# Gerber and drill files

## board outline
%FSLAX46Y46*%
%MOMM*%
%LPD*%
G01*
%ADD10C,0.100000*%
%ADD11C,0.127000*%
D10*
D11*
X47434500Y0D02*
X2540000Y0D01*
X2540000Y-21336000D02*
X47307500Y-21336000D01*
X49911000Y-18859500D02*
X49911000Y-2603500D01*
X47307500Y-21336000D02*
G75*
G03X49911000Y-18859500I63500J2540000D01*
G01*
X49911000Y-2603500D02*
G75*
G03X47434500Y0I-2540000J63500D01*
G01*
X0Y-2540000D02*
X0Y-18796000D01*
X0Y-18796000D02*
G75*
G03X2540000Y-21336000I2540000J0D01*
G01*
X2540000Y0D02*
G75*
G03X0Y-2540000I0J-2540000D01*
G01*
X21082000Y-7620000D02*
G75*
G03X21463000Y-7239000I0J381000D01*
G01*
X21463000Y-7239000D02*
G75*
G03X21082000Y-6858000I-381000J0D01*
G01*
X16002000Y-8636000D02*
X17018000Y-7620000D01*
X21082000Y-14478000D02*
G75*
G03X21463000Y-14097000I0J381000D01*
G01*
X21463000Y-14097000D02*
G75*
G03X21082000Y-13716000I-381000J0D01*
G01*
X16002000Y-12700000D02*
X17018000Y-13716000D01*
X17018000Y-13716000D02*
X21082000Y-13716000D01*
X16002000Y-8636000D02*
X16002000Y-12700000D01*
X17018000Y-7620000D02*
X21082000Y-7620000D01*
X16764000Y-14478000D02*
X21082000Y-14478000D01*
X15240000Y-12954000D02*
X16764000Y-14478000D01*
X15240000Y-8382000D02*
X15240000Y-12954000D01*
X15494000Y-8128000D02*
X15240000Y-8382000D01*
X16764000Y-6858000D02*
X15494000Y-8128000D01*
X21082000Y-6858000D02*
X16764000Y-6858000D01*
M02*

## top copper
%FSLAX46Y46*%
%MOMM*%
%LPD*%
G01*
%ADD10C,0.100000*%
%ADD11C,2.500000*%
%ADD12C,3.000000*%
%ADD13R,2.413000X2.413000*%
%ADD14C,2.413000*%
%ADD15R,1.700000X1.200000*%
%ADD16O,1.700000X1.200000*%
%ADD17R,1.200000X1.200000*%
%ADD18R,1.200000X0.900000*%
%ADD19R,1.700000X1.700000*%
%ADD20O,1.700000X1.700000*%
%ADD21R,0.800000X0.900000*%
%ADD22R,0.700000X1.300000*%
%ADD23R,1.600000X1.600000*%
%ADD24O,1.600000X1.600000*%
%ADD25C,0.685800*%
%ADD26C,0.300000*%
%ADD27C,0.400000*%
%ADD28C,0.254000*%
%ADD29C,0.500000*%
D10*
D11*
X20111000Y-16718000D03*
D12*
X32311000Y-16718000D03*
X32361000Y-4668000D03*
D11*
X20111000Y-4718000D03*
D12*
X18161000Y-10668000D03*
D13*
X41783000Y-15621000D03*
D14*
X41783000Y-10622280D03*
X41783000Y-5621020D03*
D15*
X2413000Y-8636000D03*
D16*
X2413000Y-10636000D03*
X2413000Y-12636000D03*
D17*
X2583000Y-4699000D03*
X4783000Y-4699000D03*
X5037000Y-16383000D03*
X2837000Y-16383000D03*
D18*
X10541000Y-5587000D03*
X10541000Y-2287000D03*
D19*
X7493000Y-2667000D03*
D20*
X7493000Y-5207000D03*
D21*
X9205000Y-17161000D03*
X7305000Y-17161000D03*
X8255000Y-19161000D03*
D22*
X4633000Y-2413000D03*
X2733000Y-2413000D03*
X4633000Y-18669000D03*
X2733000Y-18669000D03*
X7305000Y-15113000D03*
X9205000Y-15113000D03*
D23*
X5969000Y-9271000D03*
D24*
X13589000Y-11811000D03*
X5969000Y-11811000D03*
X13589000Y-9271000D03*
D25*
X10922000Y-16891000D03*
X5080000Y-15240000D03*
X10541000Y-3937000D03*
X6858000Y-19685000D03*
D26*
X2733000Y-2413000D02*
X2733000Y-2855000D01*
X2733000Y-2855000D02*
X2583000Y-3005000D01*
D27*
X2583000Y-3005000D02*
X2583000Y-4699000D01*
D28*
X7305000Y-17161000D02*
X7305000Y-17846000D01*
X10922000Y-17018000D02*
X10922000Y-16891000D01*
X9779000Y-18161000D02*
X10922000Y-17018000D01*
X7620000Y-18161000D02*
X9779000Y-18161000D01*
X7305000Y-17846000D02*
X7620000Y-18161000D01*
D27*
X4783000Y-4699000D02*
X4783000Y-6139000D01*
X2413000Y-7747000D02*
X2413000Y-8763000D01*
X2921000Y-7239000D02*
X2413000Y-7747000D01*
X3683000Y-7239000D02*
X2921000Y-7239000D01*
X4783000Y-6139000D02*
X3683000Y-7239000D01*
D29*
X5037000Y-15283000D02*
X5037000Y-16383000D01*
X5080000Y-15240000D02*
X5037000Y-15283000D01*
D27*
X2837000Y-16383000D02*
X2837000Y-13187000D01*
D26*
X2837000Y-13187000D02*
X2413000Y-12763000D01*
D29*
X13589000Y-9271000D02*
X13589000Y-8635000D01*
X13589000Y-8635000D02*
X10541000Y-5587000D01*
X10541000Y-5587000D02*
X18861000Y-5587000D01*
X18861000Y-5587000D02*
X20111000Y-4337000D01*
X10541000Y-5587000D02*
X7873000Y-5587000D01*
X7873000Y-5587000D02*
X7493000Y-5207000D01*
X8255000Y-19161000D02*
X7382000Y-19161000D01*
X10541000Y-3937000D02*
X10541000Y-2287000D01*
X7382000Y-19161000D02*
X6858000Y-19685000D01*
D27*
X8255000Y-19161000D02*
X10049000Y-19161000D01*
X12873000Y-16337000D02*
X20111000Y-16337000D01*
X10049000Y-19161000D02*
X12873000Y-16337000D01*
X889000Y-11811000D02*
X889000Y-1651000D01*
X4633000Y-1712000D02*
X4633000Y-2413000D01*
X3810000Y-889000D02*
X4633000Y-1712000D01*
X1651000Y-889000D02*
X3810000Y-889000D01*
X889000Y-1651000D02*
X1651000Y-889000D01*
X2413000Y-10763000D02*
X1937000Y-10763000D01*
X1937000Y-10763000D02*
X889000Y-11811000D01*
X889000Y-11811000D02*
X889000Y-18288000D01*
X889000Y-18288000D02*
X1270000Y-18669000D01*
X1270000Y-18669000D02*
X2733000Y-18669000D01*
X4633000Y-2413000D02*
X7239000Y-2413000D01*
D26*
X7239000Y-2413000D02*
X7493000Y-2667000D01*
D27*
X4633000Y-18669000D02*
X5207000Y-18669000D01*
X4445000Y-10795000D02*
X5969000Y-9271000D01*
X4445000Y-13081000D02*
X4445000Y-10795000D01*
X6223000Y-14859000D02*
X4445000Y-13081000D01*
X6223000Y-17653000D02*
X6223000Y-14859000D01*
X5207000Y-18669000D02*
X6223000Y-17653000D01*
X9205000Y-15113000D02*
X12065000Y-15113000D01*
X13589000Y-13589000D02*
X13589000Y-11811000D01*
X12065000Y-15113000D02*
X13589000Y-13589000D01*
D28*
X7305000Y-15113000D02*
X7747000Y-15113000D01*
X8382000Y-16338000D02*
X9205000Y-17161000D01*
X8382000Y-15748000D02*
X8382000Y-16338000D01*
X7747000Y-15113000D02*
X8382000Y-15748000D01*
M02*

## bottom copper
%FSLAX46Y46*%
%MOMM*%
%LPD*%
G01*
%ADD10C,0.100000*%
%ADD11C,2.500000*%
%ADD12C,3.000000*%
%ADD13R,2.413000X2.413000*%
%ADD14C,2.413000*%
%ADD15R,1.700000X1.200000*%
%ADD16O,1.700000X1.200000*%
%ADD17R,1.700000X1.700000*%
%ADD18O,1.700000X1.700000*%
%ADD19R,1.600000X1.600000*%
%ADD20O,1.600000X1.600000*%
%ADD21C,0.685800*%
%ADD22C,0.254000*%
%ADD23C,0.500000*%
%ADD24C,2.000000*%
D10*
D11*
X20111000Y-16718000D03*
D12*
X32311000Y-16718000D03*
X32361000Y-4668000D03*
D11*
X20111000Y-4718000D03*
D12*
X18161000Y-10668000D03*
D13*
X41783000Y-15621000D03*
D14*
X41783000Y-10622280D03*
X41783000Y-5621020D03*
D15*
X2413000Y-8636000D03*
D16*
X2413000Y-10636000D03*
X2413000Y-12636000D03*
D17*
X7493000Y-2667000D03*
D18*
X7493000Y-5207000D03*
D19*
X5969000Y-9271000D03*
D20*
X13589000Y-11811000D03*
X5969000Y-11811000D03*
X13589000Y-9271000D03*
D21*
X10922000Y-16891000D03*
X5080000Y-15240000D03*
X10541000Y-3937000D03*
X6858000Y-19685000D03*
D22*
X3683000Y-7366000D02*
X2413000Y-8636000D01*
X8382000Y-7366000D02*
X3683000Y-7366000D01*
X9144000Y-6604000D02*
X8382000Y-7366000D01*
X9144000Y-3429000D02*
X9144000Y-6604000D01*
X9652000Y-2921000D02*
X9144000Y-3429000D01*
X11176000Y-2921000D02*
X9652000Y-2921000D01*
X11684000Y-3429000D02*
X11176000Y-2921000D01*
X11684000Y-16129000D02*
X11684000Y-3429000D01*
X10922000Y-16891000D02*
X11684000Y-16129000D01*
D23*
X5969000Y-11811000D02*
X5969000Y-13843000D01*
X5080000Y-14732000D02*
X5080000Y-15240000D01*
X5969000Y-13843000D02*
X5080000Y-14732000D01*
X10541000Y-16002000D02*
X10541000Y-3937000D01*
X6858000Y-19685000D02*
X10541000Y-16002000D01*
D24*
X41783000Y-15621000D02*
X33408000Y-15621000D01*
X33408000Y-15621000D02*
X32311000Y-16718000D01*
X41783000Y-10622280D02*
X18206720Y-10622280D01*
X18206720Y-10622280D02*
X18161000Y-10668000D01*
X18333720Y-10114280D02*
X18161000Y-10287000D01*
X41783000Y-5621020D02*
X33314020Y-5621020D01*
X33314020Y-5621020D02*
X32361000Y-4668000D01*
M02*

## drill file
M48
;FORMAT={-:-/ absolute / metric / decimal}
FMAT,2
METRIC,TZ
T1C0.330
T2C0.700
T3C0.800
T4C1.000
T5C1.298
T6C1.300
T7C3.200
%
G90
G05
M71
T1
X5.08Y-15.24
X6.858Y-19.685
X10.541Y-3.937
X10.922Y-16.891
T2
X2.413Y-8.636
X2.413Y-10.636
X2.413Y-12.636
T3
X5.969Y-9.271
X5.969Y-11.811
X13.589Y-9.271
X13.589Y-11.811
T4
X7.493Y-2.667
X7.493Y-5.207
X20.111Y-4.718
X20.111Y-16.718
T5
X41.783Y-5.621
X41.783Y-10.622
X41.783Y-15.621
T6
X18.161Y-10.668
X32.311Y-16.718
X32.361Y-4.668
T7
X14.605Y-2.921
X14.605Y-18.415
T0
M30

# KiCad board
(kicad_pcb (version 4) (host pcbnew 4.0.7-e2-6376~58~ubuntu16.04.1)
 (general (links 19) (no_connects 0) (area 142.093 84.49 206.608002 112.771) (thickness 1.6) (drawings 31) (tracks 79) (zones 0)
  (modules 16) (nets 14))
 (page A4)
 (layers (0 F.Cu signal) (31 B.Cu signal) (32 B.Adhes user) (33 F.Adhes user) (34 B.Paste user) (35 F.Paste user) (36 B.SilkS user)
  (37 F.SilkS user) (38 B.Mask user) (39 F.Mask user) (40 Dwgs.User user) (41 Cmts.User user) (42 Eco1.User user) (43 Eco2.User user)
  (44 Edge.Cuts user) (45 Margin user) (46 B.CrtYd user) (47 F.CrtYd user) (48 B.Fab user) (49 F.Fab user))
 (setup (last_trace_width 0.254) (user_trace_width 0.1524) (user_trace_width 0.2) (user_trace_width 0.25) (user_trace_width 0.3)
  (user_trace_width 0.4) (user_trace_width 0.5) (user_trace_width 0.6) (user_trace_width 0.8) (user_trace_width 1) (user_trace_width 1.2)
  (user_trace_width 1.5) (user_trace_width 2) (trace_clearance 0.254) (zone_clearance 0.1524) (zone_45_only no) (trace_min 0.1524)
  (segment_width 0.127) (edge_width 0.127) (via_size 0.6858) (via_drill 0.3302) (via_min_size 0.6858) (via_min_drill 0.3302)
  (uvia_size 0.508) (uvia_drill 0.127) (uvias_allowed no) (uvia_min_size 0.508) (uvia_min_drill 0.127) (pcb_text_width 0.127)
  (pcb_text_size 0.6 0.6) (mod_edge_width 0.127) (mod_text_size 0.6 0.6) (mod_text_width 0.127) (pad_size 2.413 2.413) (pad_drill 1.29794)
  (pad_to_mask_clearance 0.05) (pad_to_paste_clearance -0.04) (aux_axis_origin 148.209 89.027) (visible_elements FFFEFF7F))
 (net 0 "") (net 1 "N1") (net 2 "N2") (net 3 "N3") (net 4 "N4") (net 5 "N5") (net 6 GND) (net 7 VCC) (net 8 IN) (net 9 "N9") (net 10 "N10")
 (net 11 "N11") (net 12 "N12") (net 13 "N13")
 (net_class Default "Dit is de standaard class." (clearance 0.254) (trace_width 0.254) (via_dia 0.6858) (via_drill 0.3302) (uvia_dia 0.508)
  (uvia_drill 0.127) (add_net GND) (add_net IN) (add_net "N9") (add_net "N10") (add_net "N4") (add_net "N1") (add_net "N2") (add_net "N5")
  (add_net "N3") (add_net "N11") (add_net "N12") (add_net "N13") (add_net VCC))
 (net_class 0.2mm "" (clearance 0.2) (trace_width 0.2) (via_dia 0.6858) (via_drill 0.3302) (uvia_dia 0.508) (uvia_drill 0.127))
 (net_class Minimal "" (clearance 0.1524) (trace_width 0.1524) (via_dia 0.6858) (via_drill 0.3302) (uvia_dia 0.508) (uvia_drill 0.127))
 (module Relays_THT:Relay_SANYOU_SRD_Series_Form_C (layer F.Cu) (at 166.37 99.695)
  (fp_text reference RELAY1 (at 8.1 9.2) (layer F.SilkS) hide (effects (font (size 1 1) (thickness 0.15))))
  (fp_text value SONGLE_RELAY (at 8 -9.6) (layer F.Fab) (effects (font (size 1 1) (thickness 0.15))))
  (pad 4 thru_hole circle (at 1.95 6.05 90) (size 2.5 2.5) (drill 1) (layers *.Cu *.Mask) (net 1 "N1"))
  (pad 1 thru_hole circle (at 14.15 6.05 90) (size 3 3) (drill 1.3) (layers *.Cu *.Mask) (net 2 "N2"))
  (pad 2 thru_hole circle (at 14.2 -6 90) (size 3 3) (drill 1.3) (layers *.Cu *.Mask) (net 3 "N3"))
  (pad 5 thru_hole circle (at 1.95 -5.95 90) (size 2.5 2.5) (drill 1) (layers *.Cu *.Mask) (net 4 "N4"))
  (pad 3 thru_hole circle (at 0 0 90) (size 3 3) (drill 1.3) (layers *.Cu *.Mask) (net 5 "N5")))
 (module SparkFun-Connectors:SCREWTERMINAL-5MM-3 (layer F.Cu) (at 189.992 104.648 90)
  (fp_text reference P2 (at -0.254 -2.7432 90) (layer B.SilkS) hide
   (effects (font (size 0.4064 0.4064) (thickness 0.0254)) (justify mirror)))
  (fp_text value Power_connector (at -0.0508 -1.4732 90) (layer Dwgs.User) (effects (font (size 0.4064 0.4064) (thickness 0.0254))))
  (pad 1 thru_hole rect (at 0 0 90) (size 2.413 2.413) (drill 1.29794) (layers *.Cu *.Mask F.Paste F.SilkS) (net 2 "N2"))
  (pad 2 thru_hole circle (at 4.99872 0 90) (size 2.413 2.413) (drill 1.29794) (layers *.Cu *.Mask F.Paste F.SilkS) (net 5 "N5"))
  (pad 3 thru_hole circle (at 9.99998 0 90) (size 2.413 2.413) (drill 1.29794) (layers *.Cu *.Mask F.Paste F.SilkS) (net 3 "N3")))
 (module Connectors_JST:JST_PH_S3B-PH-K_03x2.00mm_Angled (layer F.Cu) (at 150.622 97.663 270)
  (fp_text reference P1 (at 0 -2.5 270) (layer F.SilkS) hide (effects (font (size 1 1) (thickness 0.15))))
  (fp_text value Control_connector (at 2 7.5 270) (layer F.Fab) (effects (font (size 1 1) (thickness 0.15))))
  (pad 1 thru_hole rect (at 0 0 270) (size 1.2 1.7) (drill 0.7) (layers *.Cu *.Mask) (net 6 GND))
  (pad 2 thru_hole oval (at 2 0 270) (size 1.2 1.7) (drill 0.7) (layers *.Cu *.Mask) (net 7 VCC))
  (pad 3 thru_hole oval (at 4 0 270) (size 1.2 1.7) (drill 0.7) (layers *.Cu *.Mask) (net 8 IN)))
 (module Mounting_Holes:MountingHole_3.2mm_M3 (layer F.Cu) (at 162.814 107.442)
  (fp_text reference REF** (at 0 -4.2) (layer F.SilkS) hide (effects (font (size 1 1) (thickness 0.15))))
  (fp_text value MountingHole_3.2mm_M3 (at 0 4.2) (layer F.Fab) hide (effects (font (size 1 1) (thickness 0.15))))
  (pad 1 np_thru_hole circle (at 0 0) (size 3.2 3.2) (drill 3.2) (layers *.Cu *.Mask)))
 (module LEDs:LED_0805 (layer F.Cu) (at 151.892 93.726 180)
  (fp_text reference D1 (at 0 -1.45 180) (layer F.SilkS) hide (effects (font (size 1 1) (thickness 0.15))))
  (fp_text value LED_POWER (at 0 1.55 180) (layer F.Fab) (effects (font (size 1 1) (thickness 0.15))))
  (pad 2 smd rect (at 1.1 0) (size 1.2 1.2) (layers F.Cu F.Paste F.Mask) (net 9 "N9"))
  (pad 1 smd rect (at -1.1 0) (size 1.2 1.2) (layers F.Cu F.Paste F.Mask) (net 6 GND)))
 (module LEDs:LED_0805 (layer F.Cu) (at 152.146 105.41)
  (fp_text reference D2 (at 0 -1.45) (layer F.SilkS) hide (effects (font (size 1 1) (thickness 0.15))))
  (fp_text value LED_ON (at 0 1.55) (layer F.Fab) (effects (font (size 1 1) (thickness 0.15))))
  (pad 2 smd rect (at 1.1 0 180) (size 1.2 1.2) (layers F.Cu F.Paste F.Mask) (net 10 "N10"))
  (pad 1 smd rect (at -1.1 0 180) (size 1.2 1.2) (layers F.Cu F.Paste F.Mask) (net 8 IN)))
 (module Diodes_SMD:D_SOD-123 (layer F.Cu) (at 158.75 92.964 90)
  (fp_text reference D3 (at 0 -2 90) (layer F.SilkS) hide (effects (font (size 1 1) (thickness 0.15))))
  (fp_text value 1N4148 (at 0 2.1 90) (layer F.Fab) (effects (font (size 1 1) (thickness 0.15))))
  (pad 1 smd rect (at -1.65 0 90) (size 0.9 1.2) (layers F.Cu F.Paste F.Mask) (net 4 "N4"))
  (pad 2 smd rect (at 1.65 0 90) (size 0.9 1.2) (layers F.Cu F.Paste F.Mask) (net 1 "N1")))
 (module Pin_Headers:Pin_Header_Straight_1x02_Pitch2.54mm (layer F.Cu) (at 155.702 91.694)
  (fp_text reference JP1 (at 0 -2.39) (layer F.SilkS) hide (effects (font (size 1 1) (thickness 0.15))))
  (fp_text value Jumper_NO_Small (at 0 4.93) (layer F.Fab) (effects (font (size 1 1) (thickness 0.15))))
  (pad 1 thru_hole rect (at 0 0) (size 1.7 1.7) (drill 1) (layers *.Cu *.Mask) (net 7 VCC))
  (pad 2 thru_hole oval (at 0 2.54) (size 1.7 1.7) (drill 1) (layers *.Cu *.Mask) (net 4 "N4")))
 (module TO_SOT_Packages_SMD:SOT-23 (layer F.Cu) (at 156.464 107.188 270)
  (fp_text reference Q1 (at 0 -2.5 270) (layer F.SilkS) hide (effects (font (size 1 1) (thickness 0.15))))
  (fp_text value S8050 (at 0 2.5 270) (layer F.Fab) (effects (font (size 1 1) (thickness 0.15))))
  (pad 1 smd rect (at -1 -0.95 270) (size 0.9 0.8) (layers F.Cu F.Paste F.Mask) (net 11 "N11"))
  (pad 2 smd rect (at -1 0.95 270) (size 0.9 0.8) (layers F.Cu F.Paste F.Mask) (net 6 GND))
  (pad 3 smd rect (at 1 0 270) (size 0.9 0.8) (layers F.Cu F.Paste F.Mask) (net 1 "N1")))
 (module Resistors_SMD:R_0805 (layer F.Cu) (at 151.892 91.44 180)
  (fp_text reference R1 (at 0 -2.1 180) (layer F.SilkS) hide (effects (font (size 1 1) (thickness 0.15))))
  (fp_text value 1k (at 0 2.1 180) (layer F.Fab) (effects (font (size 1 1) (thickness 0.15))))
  (pad 1 smd rect (at -0.95 0 180) (size 0.7 1.3) (layers F.Cu F.Paste F.Mask) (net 7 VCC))
  (pad 2 smd rect (at 0.95 0 180) (size 0.7 1.3) (layers F.Cu F.Paste F.Mask) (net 9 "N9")))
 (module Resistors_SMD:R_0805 (layer F.Cu) (at 151.892 107.696 180)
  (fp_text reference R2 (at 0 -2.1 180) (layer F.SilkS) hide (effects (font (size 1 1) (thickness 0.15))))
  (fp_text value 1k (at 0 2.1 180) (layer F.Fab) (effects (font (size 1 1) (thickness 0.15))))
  (pad 1 smd rect (at -0.95 0 180) (size 0.7 1.3) (layers F.Cu F.Paste F.Mask) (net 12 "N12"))
  (pad 2 smd rect (at 0.95 0 180) (size 0.7 1.3) (layers F.Cu F.Paste F.Mask) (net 7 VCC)))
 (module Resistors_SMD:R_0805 (layer F.Cu) (at 156.464 104.14)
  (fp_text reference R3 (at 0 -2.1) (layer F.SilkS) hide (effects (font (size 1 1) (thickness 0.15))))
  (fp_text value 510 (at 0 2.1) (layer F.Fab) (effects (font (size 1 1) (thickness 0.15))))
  (pad 1 smd rect (at -0.95 0) (size 0.7 1.3) (layers F.Cu F.Paste F.Mask) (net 11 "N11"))
  (pad 2 smd rect (at 0.95 0) (size 0.7 1.3) (layers F.Cu F.Paste F.Mask) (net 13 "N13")))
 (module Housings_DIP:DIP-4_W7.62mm (layer F.Cu) (at 154.178 98.298)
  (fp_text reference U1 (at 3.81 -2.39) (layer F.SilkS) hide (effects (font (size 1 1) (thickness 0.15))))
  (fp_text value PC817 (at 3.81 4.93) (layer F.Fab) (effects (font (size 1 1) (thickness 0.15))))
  (pad 1 thru_hole rect (at 0 0) (size 1.6 1.6) (drill 0.8) (layers *.Cu *.Mask) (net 12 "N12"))
  (pad 3 thru_hole oval (at 7.62 2.54) (size 1.6 1.6) (drill 0.8) (layers *.Cu *.Mask) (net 13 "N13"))
  (pad 2 thru_hole oval (at 0 2.54) (size 1.6 1.6) (drill 0.8) (layers *.Cu *.Mask) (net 10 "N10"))
  (pad 4 thru_hole oval (at 7.62 0) (size 1.6 1.6) (drill 0.8) (layers *.Cu *.Mask) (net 4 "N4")))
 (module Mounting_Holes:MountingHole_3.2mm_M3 (layer F.Cu) (at 162.814 91.948)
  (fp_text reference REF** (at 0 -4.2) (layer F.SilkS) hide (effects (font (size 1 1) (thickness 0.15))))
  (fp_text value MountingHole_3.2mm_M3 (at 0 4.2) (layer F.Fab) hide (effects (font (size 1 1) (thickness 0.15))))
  (pad 1 np_thru_hole circle (at 0 0) (size 3.2 3.2) (drill 3.2) (layers *.Cu *.Mask)))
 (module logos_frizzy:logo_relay (layer B.Cu) (at 175.26 99.695 90)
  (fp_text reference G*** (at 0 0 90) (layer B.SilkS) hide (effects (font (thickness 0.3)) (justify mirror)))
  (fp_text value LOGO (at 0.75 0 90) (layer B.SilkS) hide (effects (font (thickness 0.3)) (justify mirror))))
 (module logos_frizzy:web (layer F.Cu) (at 174.371 108.712)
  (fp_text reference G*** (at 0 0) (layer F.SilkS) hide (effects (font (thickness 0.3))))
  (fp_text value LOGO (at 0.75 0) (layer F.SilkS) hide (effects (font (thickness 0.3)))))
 (gr_line (start 195.6435 89.027) (end 150.749 89.027) (angle 90) (layer Edge.Cuts) (width 0.127))
 (gr_line (start 150.749 110.363) (end 195.5165 110.363) (angle 90) (layer Edge.Cuts) (width 0.127))
 (gr_line (start 198.12 107.8865) (end 198.12 91.6305) (angle 90) (layer Edge.Cuts) (width 0.127))
 (gr_arc (start 195.58 107.823) (end 198.12 107.8865) (angle 90) (layer Edge.Cuts) (width 0.127))
 (gr_arc (start 195.58 91.567) (end 195.6435 89.027) (angle 90) (layer Edge.Cuts) (width 0.127))
 (gr_line (start 148.209 91.567) (end 148.209 107.823) (angle 90) (layer Edge.Cuts) (width 0.127))
 (gr_arc (start 150.749 107.823) (end 150.749 110.363) (angle 90) (layer Edge.Cuts) (width 0.127))
 (gr_arc (start 150.749 91.567) (end 148.209 91.567) (angle 90) (layer Edge.Cuts) (width 0.127))
 (gr_arc (start 169.291 96.266) (end 169.672 96.266) (angle 90) (layer Edge.Cuts) (width 0.127))
 (gr_arc (start 169.291 96.266) (end 169.291 95.885) (angle 90) (layer Edge.Cuts) (width 0.127))
 (gr_line (start 164.211 97.663) (end 165.227 96.647) (angle 90) (layer Edge.Cuts) (width 0.127))
 (gr_arc (start 169.291 103.124) (end 169.672 103.124) (angle 90) (layer Edge.Cuts) (width 0.127))
 (gr_arc (start 169.291 103.124) (end 169.291 102.743) (angle 90) (layer Edge.Cuts) (width 0.127))
 (gr_line (start 164.211 101.727) (end 165.227 102.743) (angle 90) (layer Edge.Cuts) (width 0.127))
 (gr_line (start 165.227 102.743) (end 169.291 102.743) (angle 90) (layer Edge.Cuts) (width 0.127))
 (gr_line (start 164.211 97.663) (end 164.211 101.727) (angle 90) (layer Edge.Cuts) (width 0.127))
 (gr_line (start 165.227 96.647) (end 169.291 96.647) (angle 90) (layer Edge.Cuts) (width 0.127))
 (gr_line (start 164.973 103.505) (end 169.291 103.505) (angle 90) (layer Edge.Cuts) (width 0.127))
 (gr_line (start 163.449 101.981) (end 164.973 103.505) (angle 90) (layer Edge.Cuts) (width 0.127))
 (gr_line (start 163.449 97.409) (end 163.449 101.981) (angle 90) (layer Edge.Cuts) (width 0.127))
 (gr_line (start 163.703 97.155) (end 163.449 97.409) (angle 90) (layer Edge.Cuts) (width 0.127))
 (gr_line (start 164.973 95.885) (end 163.703 97.155) (angle 90) (layer Edge.Cuts) (width 0.127))
 (gr_line (start 169.291 95.885) (end 164.973 95.885) (angle 90) (layer Edge.Cuts) (width 0.127))
 (segment (start 150.942 91.44) (end 150.942 91.882) (width 0.3) (layer F.Cu) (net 9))
 (segment (start 150.942 91.882) (end 150.792 92.032) (width 0.3) (layer F.Cu) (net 9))
 (segment (start 150.792 92.032) (end 150.792 93.726) (width 0.4) (layer F.Cu) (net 9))
 (segment (start 155.514 106.188) (end 155.514 106.873) (width 0.254) (layer F.Cu) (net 6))
 (segment (start 151.892 96.393) (end 150.622 97.663) (width 0.254) (layer B.Cu) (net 6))
 (segment (start 156.591 96.393) (end 151.892 96.393) (width 0.254) (layer B.Cu) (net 6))
 (segment (start 157.353 95.631) (end 156.591 96.393) (width 0.254) (layer B.Cu) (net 6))
 (segment (start 157.353 92.456) (end 157.353 95.631) (width 0.254) (layer B.Cu) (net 6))
 (segment (start 157.861 91.948) (end 157.353 92.456) (width 0.254) (layer B.Cu) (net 6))
 (segment (start 159.385 91.948) (end 157.861 91.948) (width 0.254) (layer B.Cu) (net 6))
 (segment (start 159.893 92.456) (end 159.385 91.948) (width 0.254) (layer B.Cu) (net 6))
 (segment (start 159.893 105.156) (end 159.893 92.456) (width 0.254) (layer B.Cu) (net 6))
 (segment (start 159.131 105.918) (end 159.893 105.156) (width 0.254) (layer B.Cu) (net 6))
 (via (at 159.131 105.918) (size 0.6858) (drill 0.3302) (layers F.Cu B.Cu) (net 6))
 (segment (start 159.131 106.045) (end 159.131 105.918) (width 0.254) (layer F.Cu) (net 6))
 (segment (start 157.988 107.188) (end 159.131 106.045) (width 0.254) (layer F.Cu) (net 6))
 (segment (start 155.829 107.188) (end 157.988 107.188) (width 0.254) (layer F.Cu) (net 6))
 (segment (start 155.514 106.873) (end 155.829 107.188) (width 0.254) (layer F.Cu) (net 6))
 (segment (start 152.992 93.726) (end 152.992 95.166) (width 0.4) (layer F.Cu) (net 6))
 (segment (start 150.622 96.774) (end 150.622 97.79) (width 0.4) (layer F.Cu) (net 6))
 (segment (start 151.13 96.266) (end 150.622 96.774) (width 0.4) (layer F.Cu) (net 6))
 (segment (start 151.892 96.266) (end 151.13 96.266) (width 0.4) (layer F.Cu) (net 6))
 (segment (start 152.992 95.166) (end 151.892 96.266) (width 0.4) (layer F.Cu) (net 6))
 (segment (start 154.178 100.838) (end 154.178 102.87) (width 0.5) (layer B.Cu) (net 10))
 (segment (start 153.246 104.31) (end 153.246 105.41) (width 0.5) (layer F.Cu) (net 10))
 (segment (start 153.289 104.267) (end 153.246 104.31) (width 0.5) (layer F.Cu) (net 10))
 (via (at 153.289 104.267) (size 0.6858) (drill 0.3302) (layers F.Cu B.Cu) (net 10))
 (segment (start 153.289 103.759) (end 153.289 104.267) (width 0.5) (layer B.Cu) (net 10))
 (segment (start 154.178 102.87) (end 153.289 103.759) (width 0.5) (layer B.Cu) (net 10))
 (segment (start 151.046 105.41) (end 151.046 102.214) (width 0.4) (layer F.Cu) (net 8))
 (segment (start 151.046 102.214) (end 150.622 101.79) (width 0.3) (layer F.Cu) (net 8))
 (segment (start 161.798 98.298) (end 161.798 97.662) (width 0.5) (layer F.Cu) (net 4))
 (segment (start 161.798 97.662) (end 158.75 94.614) (width 0.5) (layer F.Cu) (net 4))
 (segment (start 158.75 94.614) (end 167.07 94.614) (width 0.5) (layer F.Cu) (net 4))
 (segment (start 167.07 94.614) (end 168.32 93.364) (width 0.5) (layer F.Cu) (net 4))
 (segment (start 158.75 94.614) (end 156.082 94.614) (width 0.5) (layer F.Cu) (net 4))
 (segment (start 156.082 94.614) (end 155.702 94.234) (width 0.5) (layer F.Cu) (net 4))
 (segment (start 156.464 108.188) (end 155.591 108.188) (width 0.5) (layer F.Cu) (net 1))
 (segment (start 158.75 92.964) (end 158.75 91.314) (width 0.5) (layer F.Cu) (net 1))
 (via (at 158.75 92.964) (size 0.6858) (drill 0.3302) (layers F.Cu B.Cu) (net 1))
 (segment (start 158.75 105.029) (end 158.75 92.964) (width 0.5) (layer B.Cu) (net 1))
 (segment (start 155.067 108.712) (end 158.75 105.029) (width 0.5) (layer B.Cu) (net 1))
 (via (at 155.067 108.712) (size 0.6858) (drill 0.3302) (layers F.Cu B.Cu) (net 1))
 (segment (start 155.591 108.188) (end 155.067 108.712) (width 0.5) (layer F.Cu) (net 1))
 (segment (start 156.464 108.188) (end 158.258 108.188) (width 0.4) (layer F.Cu) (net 1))
 (segment (start 161.082 105.364) (end 168.32 105.364) (width 0.4) (layer F.Cu) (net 1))
 (segment (start 158.258 108.188) (end 161.082 105.364) (width 0.4) (layer F.Cu) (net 1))
 (segment (start 149.098 100.838) (end 149.098 90.678) (width 0.4) (layer F.Cu) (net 7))
 (segment (start 152.842 90.739) (end 152.842 91.44) (width 0.4) (layer F.Cu) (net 7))
 (segment (start 152.019 89.916) (end 152.842 90.739) (width 0.4) (layer F.Cu) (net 7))
 (segment (start 149.86 89.916) (end 152.019 89.916) (width 0.4) (layer F.Cu) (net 7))
 (segment (start 149.098 90.678) (end 149.86 89.916) (width 0.4) (layer F.Cu) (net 7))
 (segment (start 150.622 99.79) (end 150.146 99.79) (width 0.4) (layer F.Cu) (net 7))
 (segment (start 150.146 99.79) (end 149.098 100.838) (width 0.4) (layer F.Cu) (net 7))
 (segment (start 149.098 100.838) (end 149.098 107.315) (width 0.4) (layer F.Cu) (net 7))
 (segment (start 149.098 107.315) (end 149.479 107.696) (width 0.4) (layer F.Cu) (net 7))
 (segment (start 149.479 107.696) (end 150.942 107.696) (width 0.4) (layer F.Cu) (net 7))
 (segment (start 152.842 91.44) (end 155.448 91.44) (width 0.4) (layer F.Cu) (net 7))
 (segment (start 155.448 91.44) (end 155.702 91.694) (width 0.3) (layer F.Cu) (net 7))
 (segment (start 189.992 104.648) (end 181.617 104.648) (width 2) (layer B.Cu) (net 2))
 (segment (start 181.617 104.648) (end 180.52 105.745) (width 2) (layer B.Cu) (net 2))
 (segment (start 189.992 99.64928) (end 166.41572 99.64928) (width 2) (layer B.Cu) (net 5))
 (segment (start 166.41572 99.64928) (end 166.37 99.695) (width 2) (layer B.Cu) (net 5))
 (segment (start 166.54272 99.14128) (end 166.37 99.314) (width 2) (layer B.Cu) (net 5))
 (segment (start 189.992 94.64802) (end 181.52302 94.64802) (width 2) (layer B.Cu) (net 3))
 (segment (start 181.52302 94.64802) (end 180.57 93.695) (width 2) (layer B.Cu) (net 3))
 (segment (start 152.842 107.696) (end 153.416 107.696) (width 0.4) (layer F.Cu) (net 12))
 (segment (start 152.654 99.822) (end 154.178 98.298) (width 0.4) (layer F.Cu) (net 12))
 (segment (start 152.654 102.108) (end 152.654 99.822) (width 0.4) (layer F.Cu) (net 12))
 (segment (start 154.432 103.886) (end 152.654 102.108) (width 0.4) (layer F.Cu) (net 12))
 (segment (start 154.432 106.68) (end 154.432 103.886) (width 0.4) (layer F.Cu) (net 12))
 (segment (start 153.416 107.696) (end 154.432 106.68) (width 0.4) (layer F.Cu) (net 12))
 (segment (start 157.414 104.14) (end 160.274 104.14) (width 0.4) (layer F.Cu) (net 13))
 (segment (start 161.798 102.616) (end 161.798 100.838) (width 0.4) (layer F.Cu) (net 13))
 (segment (start 160.274 104.14) (end 161.798 102.616) (width 0.4) (layer F.Cu) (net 13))
 (segment (start 155.514 104.14) (end 155.956 104.14) (width 0.254) (layer F.Cu) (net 11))
 (segment (start 156.591 105.365) (end 157.414 106.188) (width 0.254) (layer F.Cu) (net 11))
 (segment (start 156.591 104.775) (end 156.591 105.365) (width 0.254) (layer F.Cu) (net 11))
 (segment (start 155.956 104.14) (end 156.591 104.775) (width 0.254) (layer F.Cu) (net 11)))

